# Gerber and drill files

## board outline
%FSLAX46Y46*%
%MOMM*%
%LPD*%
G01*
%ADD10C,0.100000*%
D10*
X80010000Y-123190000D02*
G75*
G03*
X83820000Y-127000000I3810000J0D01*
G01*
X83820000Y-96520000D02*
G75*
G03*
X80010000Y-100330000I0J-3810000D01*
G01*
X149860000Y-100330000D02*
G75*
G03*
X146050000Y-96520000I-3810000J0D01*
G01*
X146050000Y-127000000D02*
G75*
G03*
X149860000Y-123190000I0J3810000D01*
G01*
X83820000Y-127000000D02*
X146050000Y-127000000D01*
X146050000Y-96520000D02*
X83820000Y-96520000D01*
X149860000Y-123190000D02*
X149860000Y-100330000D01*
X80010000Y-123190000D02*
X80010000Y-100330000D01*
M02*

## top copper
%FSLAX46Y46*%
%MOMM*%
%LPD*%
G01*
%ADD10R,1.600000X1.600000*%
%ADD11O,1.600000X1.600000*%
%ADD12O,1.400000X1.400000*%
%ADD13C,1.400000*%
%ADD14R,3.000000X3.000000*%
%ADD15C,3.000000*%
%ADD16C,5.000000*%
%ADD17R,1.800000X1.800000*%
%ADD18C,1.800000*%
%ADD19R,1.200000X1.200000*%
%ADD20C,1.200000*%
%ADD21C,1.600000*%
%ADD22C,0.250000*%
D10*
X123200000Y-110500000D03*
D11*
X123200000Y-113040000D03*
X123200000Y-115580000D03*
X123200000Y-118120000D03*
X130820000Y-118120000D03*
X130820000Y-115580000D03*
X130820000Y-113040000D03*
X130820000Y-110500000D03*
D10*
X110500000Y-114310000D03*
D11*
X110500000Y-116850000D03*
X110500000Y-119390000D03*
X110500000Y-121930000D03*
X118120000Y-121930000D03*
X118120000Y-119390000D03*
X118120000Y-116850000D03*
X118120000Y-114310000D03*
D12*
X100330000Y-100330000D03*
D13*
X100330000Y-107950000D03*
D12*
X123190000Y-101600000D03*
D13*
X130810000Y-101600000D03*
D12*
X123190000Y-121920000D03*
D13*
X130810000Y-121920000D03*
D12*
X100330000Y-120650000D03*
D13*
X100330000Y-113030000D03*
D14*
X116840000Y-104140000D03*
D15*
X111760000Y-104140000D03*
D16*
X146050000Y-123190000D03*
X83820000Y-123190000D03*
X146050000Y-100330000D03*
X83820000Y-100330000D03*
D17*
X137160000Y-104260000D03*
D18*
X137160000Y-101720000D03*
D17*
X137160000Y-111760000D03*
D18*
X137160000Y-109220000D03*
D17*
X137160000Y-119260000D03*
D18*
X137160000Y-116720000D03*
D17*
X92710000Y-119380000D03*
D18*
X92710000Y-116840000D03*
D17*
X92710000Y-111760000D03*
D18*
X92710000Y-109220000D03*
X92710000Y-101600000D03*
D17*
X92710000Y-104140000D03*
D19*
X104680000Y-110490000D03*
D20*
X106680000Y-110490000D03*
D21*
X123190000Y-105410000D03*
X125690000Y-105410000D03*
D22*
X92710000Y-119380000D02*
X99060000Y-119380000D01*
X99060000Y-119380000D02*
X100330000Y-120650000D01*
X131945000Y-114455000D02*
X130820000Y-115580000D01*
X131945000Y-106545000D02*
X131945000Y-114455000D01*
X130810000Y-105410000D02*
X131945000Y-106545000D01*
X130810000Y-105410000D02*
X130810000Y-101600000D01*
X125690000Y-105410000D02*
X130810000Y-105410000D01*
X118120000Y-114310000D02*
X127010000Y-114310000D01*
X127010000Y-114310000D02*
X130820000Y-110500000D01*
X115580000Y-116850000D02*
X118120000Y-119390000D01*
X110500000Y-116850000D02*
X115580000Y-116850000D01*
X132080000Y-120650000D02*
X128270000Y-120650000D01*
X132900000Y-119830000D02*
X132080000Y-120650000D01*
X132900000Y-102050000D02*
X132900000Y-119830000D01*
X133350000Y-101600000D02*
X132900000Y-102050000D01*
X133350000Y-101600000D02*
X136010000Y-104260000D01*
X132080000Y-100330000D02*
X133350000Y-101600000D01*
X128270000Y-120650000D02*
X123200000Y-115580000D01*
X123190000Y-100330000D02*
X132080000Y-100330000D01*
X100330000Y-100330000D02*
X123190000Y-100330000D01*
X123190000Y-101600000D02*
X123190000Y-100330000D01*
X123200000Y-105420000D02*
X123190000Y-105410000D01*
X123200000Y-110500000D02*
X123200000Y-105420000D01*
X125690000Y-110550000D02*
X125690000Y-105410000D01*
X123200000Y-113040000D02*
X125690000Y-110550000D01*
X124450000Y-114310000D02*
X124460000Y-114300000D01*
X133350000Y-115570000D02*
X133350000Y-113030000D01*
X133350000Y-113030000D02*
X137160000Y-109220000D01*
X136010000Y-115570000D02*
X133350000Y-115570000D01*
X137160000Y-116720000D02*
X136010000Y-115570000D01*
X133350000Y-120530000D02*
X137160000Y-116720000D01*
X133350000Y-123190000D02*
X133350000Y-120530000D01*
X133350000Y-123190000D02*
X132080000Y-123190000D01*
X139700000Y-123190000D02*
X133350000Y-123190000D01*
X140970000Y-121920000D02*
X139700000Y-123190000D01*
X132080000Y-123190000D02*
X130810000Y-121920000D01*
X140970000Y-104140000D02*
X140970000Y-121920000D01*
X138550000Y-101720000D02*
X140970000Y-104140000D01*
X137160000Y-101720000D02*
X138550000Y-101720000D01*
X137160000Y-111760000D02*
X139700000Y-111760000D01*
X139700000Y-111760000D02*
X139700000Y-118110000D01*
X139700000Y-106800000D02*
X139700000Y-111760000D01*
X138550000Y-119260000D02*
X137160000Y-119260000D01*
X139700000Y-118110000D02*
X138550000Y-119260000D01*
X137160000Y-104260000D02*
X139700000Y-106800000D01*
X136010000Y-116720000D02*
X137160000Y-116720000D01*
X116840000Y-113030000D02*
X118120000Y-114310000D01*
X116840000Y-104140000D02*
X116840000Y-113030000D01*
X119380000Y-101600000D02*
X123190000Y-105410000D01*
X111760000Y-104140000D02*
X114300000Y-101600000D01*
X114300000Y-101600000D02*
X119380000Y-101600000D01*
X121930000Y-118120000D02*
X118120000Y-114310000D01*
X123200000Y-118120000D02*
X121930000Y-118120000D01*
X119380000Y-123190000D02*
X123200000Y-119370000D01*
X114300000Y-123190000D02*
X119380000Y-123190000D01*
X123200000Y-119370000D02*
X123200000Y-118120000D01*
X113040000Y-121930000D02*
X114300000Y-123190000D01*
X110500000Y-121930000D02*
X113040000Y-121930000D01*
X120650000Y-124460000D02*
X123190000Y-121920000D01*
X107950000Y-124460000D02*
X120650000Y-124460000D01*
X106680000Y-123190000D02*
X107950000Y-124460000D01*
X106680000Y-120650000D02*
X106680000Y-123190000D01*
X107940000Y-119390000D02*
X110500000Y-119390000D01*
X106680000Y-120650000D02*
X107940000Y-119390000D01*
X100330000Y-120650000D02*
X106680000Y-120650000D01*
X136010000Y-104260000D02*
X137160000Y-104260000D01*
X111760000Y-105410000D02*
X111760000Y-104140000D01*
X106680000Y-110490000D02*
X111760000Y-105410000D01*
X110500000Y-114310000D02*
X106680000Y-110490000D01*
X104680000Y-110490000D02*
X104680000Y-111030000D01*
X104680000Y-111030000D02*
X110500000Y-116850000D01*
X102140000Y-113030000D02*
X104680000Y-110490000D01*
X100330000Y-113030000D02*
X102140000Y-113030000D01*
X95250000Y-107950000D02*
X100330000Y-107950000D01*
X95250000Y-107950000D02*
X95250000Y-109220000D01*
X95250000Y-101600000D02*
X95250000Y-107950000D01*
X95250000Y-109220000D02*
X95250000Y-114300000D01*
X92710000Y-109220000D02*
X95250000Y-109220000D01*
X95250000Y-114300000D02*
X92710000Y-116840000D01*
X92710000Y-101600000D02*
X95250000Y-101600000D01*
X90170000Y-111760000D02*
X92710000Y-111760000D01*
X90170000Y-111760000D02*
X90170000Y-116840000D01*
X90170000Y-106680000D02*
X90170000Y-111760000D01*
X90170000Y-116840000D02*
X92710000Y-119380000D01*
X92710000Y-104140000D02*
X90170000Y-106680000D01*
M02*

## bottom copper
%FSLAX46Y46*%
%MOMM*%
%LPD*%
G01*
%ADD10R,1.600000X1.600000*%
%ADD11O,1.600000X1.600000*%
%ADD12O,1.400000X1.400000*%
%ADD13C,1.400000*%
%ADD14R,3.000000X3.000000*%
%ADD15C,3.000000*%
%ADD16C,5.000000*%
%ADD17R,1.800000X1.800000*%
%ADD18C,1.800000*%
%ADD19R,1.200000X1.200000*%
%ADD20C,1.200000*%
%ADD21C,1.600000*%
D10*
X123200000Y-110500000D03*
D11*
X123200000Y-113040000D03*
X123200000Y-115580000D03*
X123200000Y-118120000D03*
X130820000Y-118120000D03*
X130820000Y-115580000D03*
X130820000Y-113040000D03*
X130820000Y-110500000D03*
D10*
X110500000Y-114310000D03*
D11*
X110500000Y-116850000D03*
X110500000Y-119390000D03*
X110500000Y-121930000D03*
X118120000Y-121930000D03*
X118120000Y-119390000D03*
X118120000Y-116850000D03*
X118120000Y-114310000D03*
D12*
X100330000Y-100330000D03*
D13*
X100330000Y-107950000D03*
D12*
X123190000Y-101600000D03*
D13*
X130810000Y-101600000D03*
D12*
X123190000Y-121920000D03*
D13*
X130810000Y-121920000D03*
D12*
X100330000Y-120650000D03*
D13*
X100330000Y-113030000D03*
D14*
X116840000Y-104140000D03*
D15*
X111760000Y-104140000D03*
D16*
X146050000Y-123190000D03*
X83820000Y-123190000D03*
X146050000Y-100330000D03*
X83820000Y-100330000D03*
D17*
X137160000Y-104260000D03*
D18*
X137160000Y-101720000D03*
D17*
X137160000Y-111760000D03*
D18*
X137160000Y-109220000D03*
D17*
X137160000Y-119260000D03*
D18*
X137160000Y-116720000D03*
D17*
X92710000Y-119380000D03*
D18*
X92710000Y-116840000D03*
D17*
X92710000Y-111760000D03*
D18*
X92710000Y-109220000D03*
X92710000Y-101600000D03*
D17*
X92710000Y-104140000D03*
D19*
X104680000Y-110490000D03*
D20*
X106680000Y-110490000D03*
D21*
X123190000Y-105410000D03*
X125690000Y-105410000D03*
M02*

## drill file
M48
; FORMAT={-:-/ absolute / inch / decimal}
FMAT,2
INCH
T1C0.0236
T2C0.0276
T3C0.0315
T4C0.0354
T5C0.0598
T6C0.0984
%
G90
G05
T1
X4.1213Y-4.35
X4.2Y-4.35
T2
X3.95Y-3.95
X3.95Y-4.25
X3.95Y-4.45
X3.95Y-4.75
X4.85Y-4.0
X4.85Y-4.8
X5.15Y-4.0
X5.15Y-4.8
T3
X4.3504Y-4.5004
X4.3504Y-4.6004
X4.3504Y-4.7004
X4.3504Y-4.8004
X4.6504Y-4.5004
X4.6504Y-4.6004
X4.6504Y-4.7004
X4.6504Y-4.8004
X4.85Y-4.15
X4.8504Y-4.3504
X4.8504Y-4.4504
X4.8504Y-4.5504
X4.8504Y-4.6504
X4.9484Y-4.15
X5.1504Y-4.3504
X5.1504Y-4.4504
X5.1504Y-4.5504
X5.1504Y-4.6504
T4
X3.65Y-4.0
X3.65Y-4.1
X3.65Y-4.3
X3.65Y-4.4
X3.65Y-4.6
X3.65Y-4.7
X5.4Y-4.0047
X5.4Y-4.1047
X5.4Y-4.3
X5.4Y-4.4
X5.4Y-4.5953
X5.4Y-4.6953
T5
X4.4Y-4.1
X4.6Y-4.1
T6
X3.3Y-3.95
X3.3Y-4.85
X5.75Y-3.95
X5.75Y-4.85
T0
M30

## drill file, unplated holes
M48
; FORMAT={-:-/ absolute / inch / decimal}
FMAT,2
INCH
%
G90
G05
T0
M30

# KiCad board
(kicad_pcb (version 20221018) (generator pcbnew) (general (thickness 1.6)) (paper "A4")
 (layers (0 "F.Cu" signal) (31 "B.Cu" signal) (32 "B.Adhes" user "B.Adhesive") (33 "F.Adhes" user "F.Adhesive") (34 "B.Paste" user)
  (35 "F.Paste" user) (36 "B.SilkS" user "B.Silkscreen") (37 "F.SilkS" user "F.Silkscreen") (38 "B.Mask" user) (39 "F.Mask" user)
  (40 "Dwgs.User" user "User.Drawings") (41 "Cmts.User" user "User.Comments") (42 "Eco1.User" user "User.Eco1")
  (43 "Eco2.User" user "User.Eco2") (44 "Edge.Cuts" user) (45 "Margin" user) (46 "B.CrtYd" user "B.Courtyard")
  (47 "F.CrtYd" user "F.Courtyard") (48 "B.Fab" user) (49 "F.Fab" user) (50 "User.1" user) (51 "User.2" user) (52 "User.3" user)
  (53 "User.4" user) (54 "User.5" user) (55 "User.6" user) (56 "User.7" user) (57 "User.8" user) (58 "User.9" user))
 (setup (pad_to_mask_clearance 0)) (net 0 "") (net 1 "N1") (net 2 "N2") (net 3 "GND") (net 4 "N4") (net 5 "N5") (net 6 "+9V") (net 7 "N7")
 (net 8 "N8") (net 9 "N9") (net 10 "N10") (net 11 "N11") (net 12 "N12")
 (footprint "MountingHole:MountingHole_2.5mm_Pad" (layer "F.Cu") (at 83.82 100.33)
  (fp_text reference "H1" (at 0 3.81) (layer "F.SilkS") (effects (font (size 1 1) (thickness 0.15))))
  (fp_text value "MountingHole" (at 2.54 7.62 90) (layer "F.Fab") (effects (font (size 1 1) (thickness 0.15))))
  (pad "1" thru_hole circle (at 0 0) (size 5 5) (drill 2.5) (layers "*.Cu" "*.Mask")))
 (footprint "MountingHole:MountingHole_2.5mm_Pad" (layer "F.Cu") (at 146.05 123.19)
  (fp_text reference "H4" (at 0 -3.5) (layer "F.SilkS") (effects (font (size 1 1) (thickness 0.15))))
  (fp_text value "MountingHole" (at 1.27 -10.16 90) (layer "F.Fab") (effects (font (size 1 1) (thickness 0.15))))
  (pad "1" thru_hole circle (at 0 0) (size 5 5) (drill 2.5) (layers "*.Cu" "*.Mask")))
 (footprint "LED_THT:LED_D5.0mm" (layer "F.Cu") (at 137.16 104.26 90)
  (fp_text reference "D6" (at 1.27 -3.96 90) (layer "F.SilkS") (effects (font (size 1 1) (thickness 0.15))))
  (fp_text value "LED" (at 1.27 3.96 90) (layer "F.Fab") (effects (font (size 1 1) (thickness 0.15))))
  (pad "1" thru_hole rect (at 0 0 90) (size 1.8 1.8) (drill 0.9) (layers "*.Cu" "*.Mask") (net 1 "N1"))
  (pad "2" thru_hole circle (at 2.54 0 90) (size 1.8 1.8) (drill 0.9) (layers "*.Cu" "*.Mask") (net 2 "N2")))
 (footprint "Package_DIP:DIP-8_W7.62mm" (layer "F.Cu") (at 110.5 114.31)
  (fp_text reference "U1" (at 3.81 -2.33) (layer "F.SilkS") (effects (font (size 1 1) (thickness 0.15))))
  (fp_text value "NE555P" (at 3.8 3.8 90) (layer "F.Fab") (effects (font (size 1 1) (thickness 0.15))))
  (pad "1" thru_hole rect (at 0 0) (size 1.6 1.6) (drill 0.8) (layers "*.Cu" "*.Mask") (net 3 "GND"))
  (pad "2" thru_hole oval (at 0 2.54) (size 1.6 1.6) (drill 0.8) (layers "*.Cu" "*.Mask") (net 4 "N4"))
  (pad "3" thru_hole oval (at 0 5.08) (size 1.6 1.6) (drill 0.8) (layers "*.Cu" "*.Mask") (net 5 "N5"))
  (pad "4" thru_hole oval (at 0 7.62) (size 1.6 1.6) (drill 0.8) (layers "*.Cu" "*.Mask") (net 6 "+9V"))
  (pad "5" thru_hole oval (at 7.62 7.62) (size 1.6 1.6) (drill 0.8) (layers "*.Cu" "*.Mask") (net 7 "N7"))
  (pad "6" thru_hole oval (at 7.62 5.08) (size 1.6 1.6) (drill 0.8) (layers "*.Cu" "*.Mask") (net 4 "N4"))
  (pad "7" thru_hole oval (at 7.62 2.54) (size 1.6 1.6) (drill 0.8) (layers "*.Cu" "*.Mask") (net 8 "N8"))
  (pad "8" thru_hole oval (at 7.62 0) (size 1.6 1.6) (drill 0.8) (layers "*.Cu" "*.Mask") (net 6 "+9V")))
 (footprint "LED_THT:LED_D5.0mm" (layer "F.Cu") (at 92.71 104.14 90)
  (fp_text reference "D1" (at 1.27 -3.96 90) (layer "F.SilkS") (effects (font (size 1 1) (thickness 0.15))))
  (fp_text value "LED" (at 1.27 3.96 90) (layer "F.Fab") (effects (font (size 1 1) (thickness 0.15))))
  (pad "1" thru_hole rect (at 0 0 90) (size 1.8 1.8) (drill 0.9) (layers "*.Cu" "*.Mask") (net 5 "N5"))
  (pad "2" thru_hole circle (at 2.54 0 90) (size 1.8 1.8) (drill 0.9) (layers "*.Cu" "*.Mask") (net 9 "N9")))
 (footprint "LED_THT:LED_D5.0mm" (layer "F.Cu") (at 92.71 119.38 90)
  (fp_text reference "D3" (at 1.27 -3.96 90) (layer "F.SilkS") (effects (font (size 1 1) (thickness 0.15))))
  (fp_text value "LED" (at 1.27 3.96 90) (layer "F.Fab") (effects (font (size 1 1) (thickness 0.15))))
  (pad "1" thru_hole rect (at 0 0 90) (size 1.8 1.8) (drill 0.9) (layers "*.Cu" "*.Mask") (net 5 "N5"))
  (pad "2" thru_hole circle (at 2.54 0 90) (size 1.8 1.8) (drill 0.9) (layers "*.Cu" "*.Mask") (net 9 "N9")))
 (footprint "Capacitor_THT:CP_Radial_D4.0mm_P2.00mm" (layer "F.Cu") (at 104.68 110.49)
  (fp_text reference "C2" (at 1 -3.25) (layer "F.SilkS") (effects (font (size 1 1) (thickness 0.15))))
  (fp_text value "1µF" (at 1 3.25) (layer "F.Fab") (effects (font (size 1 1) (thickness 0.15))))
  (pad "1" thru_hole rect (at 0 0) (size 1.2 1.2) (drill 0.6) (layers "*.Cu" "*.Mask") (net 4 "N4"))
  (pad "2" thru_hole circle (at 2 0) (size 1.2 1.2) (drill 0.6) (layers "*.Cu" "*.Mask") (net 3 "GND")))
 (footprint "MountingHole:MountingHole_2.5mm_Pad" (layer "F.Cu") (at 83.82 123.19)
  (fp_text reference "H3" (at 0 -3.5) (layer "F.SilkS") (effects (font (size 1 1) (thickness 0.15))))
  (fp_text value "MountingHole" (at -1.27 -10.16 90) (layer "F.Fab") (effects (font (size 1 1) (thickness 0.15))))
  (pad "1" thru_hole circle (at 0 0) (size 5 5) (drill 2.5) (layers "*.Cu" "*.Mask")))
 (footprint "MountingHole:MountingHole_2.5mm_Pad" (layer "F.Cu") (at 146.05 100.33)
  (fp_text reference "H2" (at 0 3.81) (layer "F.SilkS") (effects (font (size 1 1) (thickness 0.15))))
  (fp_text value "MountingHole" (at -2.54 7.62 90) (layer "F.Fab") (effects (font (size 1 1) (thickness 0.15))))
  (pad "1" thru_hole circle (at 0 0) (size 5 5) (drill 2.5) (layers "*.Cu" "*.Mask")))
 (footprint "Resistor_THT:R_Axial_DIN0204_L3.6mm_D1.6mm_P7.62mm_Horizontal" (layer "F.Cu") (at 100.33 113.03 -90)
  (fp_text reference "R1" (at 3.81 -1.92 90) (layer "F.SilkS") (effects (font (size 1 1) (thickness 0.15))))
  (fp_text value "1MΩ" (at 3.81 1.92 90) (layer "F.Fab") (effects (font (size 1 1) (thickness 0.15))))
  (pad "1" thru_hole circle (at 0 0 270) (size 1.4 1.4) (drill 0.7) (layers "*.Cu" "*.Mask") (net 4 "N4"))
  (pad "2" thru_hole oval (at 7.62 0 270) (size 1.4 1.4) (drill 0.7) (layers "*.Cu" "*.Mask") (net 5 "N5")))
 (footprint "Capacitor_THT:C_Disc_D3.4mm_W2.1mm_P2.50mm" (layer "F.Cu") (at 125.69 105.41 180)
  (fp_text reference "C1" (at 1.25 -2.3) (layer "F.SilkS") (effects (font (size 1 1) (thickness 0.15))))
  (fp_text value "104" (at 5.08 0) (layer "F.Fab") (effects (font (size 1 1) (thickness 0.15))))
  (pad "1" thru_hole circle (at 0 0 180) (size 1.6 1.6) (drill 0.8) (layers "*.Cu" "*.Mask") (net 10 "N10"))
  (pad "2" thru_hole circle (at 2.5 0 180) (size 1.6 1.6) (drill 0.8) (layers "*.Cu" "*.Mask") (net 3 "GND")))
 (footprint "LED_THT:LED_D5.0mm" (layer "F.Cu") (at 92.71 111.76 90)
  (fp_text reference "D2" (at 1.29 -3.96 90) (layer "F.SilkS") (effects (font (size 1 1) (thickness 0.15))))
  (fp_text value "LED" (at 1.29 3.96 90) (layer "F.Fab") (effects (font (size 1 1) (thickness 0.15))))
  (pad "1" thru_hole rect (at 0 0 90) (size 1.8 1.8) (drill 0.9) (layers "*.Cu" "*.Mask") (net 5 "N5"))
  (pad "2" thru_hole circle (at 2.54 0 90) (size 1.8 1.8) (drill 0.9) (layers "*.Cu" "*.Mask") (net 9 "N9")))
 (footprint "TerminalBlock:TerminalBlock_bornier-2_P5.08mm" (layer "F.Cu") (at 116.84 104.14 180)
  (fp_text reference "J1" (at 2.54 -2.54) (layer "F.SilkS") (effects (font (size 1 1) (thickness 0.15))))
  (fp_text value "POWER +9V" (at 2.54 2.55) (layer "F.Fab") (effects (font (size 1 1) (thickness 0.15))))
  (pad "1" thru_hole rect (at 0 0 180) (size 3 3) (drill 1.52) (layers "*.Cu" "*.Mask") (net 6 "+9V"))
  (pad "2" thru_hole circle (at 5.08 0 180) (size 3 3) (drill 1.52) (layers "*.Cu" "*.Mask") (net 3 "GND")))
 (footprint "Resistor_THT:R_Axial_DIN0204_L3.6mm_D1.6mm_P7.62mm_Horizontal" (layer "F.Cu") (at 100.33 107.95 90)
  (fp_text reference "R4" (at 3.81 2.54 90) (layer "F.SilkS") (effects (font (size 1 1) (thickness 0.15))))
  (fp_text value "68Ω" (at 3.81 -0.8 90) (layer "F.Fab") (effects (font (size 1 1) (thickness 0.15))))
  (pad "1" thru_hole circle (at 0 0 90) (size 1.4 1.4) (drill 0.7) (layers "*.Cu" "*.Mask") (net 9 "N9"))
  (pad "2" thru_hole oval (at 7.62 0 90) (size 1.4 1.4) (drill 0.7) (layers "*.Cu" "*.Mask") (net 1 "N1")))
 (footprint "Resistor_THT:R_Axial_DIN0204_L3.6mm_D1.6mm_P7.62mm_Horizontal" (layer "F.Cu") (at 130.81 101.6 180)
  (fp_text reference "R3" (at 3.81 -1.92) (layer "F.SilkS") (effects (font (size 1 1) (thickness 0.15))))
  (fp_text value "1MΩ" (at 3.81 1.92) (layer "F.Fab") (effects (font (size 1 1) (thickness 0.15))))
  (pad "1" thru_hole circle (at 0 0 180) (size 1.4 1.4) (drill 0.7) (layers "*.Cu" "*.Mask") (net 10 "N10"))
  (pad "2" thru_hole oval (at 7.62 0 180) (size 1.4 1.4) (drill 0.7) (layers "*.Cu" "*.Mask") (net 1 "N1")))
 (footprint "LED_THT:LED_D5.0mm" (layer "F.Cu") (at 137.16 119.26 90)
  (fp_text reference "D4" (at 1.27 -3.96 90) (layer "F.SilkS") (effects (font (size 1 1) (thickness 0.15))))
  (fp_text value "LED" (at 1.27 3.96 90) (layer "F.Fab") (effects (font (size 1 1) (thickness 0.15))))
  (pad "1" thru_hole rect (at 0 0 90) (size 1.8 1.8) (drill 0.9) (layers "*.Cu" "*.Mask") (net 1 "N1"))
  (pad "2" thru_hole circle (at 2.54 0 90) (size 1.8 1.8) (drill 0.9) (layers "*.Cu" "*.Mask") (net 2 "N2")))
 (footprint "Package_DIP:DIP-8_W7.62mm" (layer "F.Cu") (at 123.2 110.5)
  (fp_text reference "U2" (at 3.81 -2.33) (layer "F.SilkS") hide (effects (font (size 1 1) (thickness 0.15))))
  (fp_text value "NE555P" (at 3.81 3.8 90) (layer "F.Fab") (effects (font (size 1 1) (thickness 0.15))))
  (pad "1" thru_hole rect (at 0 0) (size 1.6 1.6) (drill 0.8) (layers "*.Cu" "*.Mask") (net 3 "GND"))
  (pad "2" thru_hole oval (at 0 2.54) (size 1.6 1.6) (drill 0.8) (layers "*.Cu" "*.Mask") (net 10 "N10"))
  (pad "3" thru_hole oval (at 0 5.08) (size 1.6 1.6) (drill 0.8) (layers "*.Cu" "*.Mask") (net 1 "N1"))
  (pad "4" thru_hole oval (at 0 7.62) (size 1.6 1.6) (drill 0.8) (layers "*.Cu" "*.Mask") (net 6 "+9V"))
  (pad "5" thru_hole oval (at 7.62 7.62) (size 1.6 1.6) (drill 0.8) (layers "*.Cu" "*.Mask") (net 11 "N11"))
  (pad "6" thru_hole oval (at 7.62 5.08) (size 1.6 1.6) (drill 0.8) (layers "*.Cu" "*.Mask") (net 10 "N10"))
  (pad "7" thru_hole oval (at 7.62 2.54) (size 1.6 1.6) (drill 0.8) (layers "*.Cu" "*.Mask") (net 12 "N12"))
  (pad "8" thru_hole oval (at 7.62 0) (size 1.6 1.6) (drill 0.8) (layers "*.Cu" "*.Mask") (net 6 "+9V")))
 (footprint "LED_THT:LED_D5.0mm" (layer "F.Cu") (at 137.16 111.76 90)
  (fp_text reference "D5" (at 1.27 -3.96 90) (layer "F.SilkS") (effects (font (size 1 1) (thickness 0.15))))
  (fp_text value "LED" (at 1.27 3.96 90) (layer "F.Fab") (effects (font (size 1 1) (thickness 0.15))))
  (pad "1" thru_hole rect (at 0 0 90) (size 1.8 1.8) (drill 0.9) (layers "*.Cu" "*.Mask") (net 1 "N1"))
  (pad "2" thru_hole circle (at 2.54 0 90) (size 1.8 1.8) (drill 0.9) (layers "*.Cu" "*.Mask") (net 2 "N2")))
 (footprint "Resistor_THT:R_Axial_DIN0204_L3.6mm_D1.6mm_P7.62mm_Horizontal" (layer "F.Cu") (at 130.81 121.92 180)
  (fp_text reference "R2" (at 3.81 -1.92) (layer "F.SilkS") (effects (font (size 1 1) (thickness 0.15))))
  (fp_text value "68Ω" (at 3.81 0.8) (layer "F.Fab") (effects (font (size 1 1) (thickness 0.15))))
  (pad "1" thru_hole circle (at 0 0 180) (size 1.4 1.4) (drill 0.7) (layers "*.Cu" "*.Mask") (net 2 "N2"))
  (pad "2" thru_hole oval (at 7.62 0 180) (size 1.4 1.4) (drill 0.7) (layers "*.Cu" "*.Mask") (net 5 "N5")))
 (gr_line (start 149.86 123.19) (end 149.86 100.33) (stroke (width 0.1) (type default)) (layer "Edge.Cuts"))
 (gr_arc (start 80.01 100.33) (mid 81.125923 97.635923) (end 83.82 96.52) (stroke (width 0.1) (type default)) (layer "Edge.Cuts"))
 (gr_arc (start 146.05 96.52) (mid 148.744077 97.635923) (end 149.86 100.33) (stroke (width 0.1) (type default)) (layer "Edge.Cuts"))
 (gr_line (start 146.05 96.52) (end 83.82 96.52) (stroke (width 0.1) (type default)) (layer "Edge.Cuts"))
 (gr_arc (start 149.86 123.19) (mid 148.744077 125.884077) (end 146.05 127) (stroke (width 0.1) (type default)) (layer "Edge.Cuts"))
 (gr_arc (start 83.82 127) (mid 81.125923 125.884077) (end 80.01 123.19) (stroke (width 0.1) (type default)) (layer "Edge.Cuts"))
 (gr_line (start 80.01 123.19) (end 80.01 100.33) (stroke (width 0.1) (type default)) (layer "Edge.Cuts"))
 (gr_line (start 83.82 127) (end 146.05 127) (stroke (width 0.1) (type default)) (layer "Edge.Cuts"))
 (segment (start 123.2 113.04) (end 125.69 110.55) (width 0.25) (layer "F.Cu") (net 10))
 (segment (start 130.81 105.41) (end 130.81 101.6) (width 0.25) (layer "F.Cu") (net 10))
 (segment (start 125.69 110.55) (end 125.69 105.41) (width 0.25) (layer "F.Cu") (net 10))
 (segment (start 125.69 105.41) (end 130.81 105.41) (width 0.25) (layer "F.Cu") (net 10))
 (segment (start 131.945 106.545) (end 131.945 114.455) (width 0.25) (layer "F.Cu") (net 10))
 (segment (start 130.81 105.41) (end 131.945 106.545) (width 0.25) (layer "F.Cu") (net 10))
 (segment (start 131.945 114.455) (end 130.82 115.58) (width 0.25) (layer "F.Cu") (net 10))
 (segment (start 111.76 105.41) (end 111.76 104.14) (width 0.25) (layer "F.Cu") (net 3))
 (segment (start 110.5 114.31) (end 106.68 110.49) (width 0.25) (layer "F.Cu") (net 3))
 (segment (start 123.2 105.42) (end 123.19 105.41) (width 0.25) (layer "F.Cu") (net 3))
 (segment (start 123.2 110.5) (end 123.2 105.42) (width 0.25) (layer "F.Cu") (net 3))
 (segment (start 114.3 101.6) (end 119.38 101.6) (width 0.25) (layer "F.Cu") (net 3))
 (segment (start 111.76 104.14) (end 114.3 101.6) (width 0.25) (layer "F.Cu") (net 3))
 (segment (start 119.38 101.6) (end 123.19 105.41) (width 0.25) (layer "F.Cu") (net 3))
 (segment (start 106.68 110.49) (end 111.76 105.41) (width 0.25) (layer "F.Cu") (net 3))
 (segment (start 115.58 116.85) (end 118.12 119.39) (width 0.25) (layer "F.Cu") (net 4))
 (segment (start 102.14 113.03) (end 104.68 110.49) (width 0.25) (layer "F.Cu") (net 4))
 (segment (start 100.33 113.03) (end 102.14 113.03) (width 0.25) (layer "F.Cu") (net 4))
 (segment (start 104.68 111.03) (end 110.5 116.85) (width 0.25) (layer "F.Cu") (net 4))
 (segment (start 104.68 110.49) (end 104.68 111.03) (width 0.25) (layer "F.Cu") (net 4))
 (segment (start 110.5 116.85) (end 115.58 116.85) (width 0.25) (layer "F.Cu") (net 4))
 (segment (start 90.17 106.68) (end 90.17 111.76) (width 0.25) (layer "F.Cu") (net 5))
 (segment (start 90.17 116.84) (end 92.71 119.38) (width 0.25) (layer "F.Cu") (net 5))
 (segment (start 90.17 111.76) (end 90.17 116.84) (width 0.25) (layer "F.Cu") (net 5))
 (segment (start 107.94 119.39) (end 110.5 119.39) (width 0.25) (layer "F.Cu") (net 5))
 (segment (start 120.65 124.46) (end 123.19 121.92) (width 0.25) (layer "F.Cu") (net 5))
 (segment (start 106.68 120.65) (end 106.68 123.19) (width 0.25) (layer "F.Cu") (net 5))
 (segment (start 92.71 119.38) (end 99.06 119.38) (width 0.25) (layer "F.Cu") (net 5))
 (segment (start 106.68 123.19) (end 107.95 124.46) (width 0.25) (layer "F.Cu") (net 5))
 (segment (start 107.95 124.46) (end 120.65 124.46) (width 0.25) (layer "F.Cu") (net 5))
 (segment (start 99.06 119.38) (end 100.33 120.65) (width 0.25) (layer "F.Cu") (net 5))
 (segment (start 92.71 104.14) (end 90.17 106.68) (width 0.25) (layer "F.Cu") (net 5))
 (segment (start 106.68 120.65) (end 107.94 119.39) (width 0.25) (layer "F.Cu") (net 5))
 (segment (start 100.33 120.65) (end 106.68 120.65) (width 0.25) (layer "F.Cu") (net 5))
 (segment (start 90.17 111.76) (end 92.71 111.76) (width 0.25) (layer "F.Cu") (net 5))
 (segment (start 95.25 109.22) (end 95.25 114.3) (width 0.25) (layer "F.Cu") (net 9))
 (segment (start 95.25 107.95) (end 95.25 109.22) (width 0.25) (layer "F.Cu") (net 9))
 (segment (start 95.25 114.3) (end 92.71 116.84) (width 0.25) (layer "F.Cu") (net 9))
 (segment (start 92.71 109.22) (end 95.25 109.22) (width 0.25) (layer "F.Cu") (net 9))
 (segment (start 92.71 101.6) (end 95.25 101.6) (width 0.25) (layer "F.Cu") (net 9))
 (segment (start 95.25 107.95) (end 100.33 107.95) (width 0.25) (layer "F.Cu") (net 9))
 (segment (start 95.25 101.6) (end 95.25 107.95) (width 0.25) (layer "F.Cu") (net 9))
 (segment (start 133.35 101.6) (end 132.9 102.05) (width 0.25) (layer "F.Cu") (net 1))
 (segment (start 123.19 100.33) (end 132.08 100.33) (width 0.25) (layer "F.Cu") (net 1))
 (segment (start 137.16 111.76) (end 139.7 111.76) (width 0.25) (layer "F.Cu") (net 1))
 (segment (start 132.08 100.33) (end 133.35 101.6) (width 0.25) (layer "F.Cu") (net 1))
 (segment (start 139.7 106.8) (end 139.7 111.76) (width 0.25) (layer "F.Cu") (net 1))
 (segment (start 139.7 111.76) (end 139.7 118.11) (width 0.25) (layer "F.Cu") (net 1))
 (segment (start 132.08 120.65) (end 128.27 120.65) (width 0.25) (layer "F.Cu") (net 1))
 (segment (start 138.55 119.26) (end 137.16 119.26) (width 0.25) (layer "F.Cu") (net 1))
 (segment (start 132.9 119.83) (end 132.08 120.65) (width 0.25) (layer "F.Cu") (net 1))
 (segment (start 128.27 120.65) (end 123.2 115.58) (width 0.25) (layer "F.Cu") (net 1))
 (segment (start 137.16 104.26) (end 139.7 106.8) (width 0.25) (layer "F.Cu") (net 1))
 (segment (start 132.9 102.05) (end 132.9 119.83) (width 0.25) (layer "F.Cu") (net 1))
 (segment (start 100.33 100.33) (end 123.19 100.33) (width 0.25) (layer "F.Cu") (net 1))
 (segment (start 136.01 104.26) (end 137.16 104.26) (width 0.25) (layer "F.Cu") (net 1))
 (segment (start 133.35 101.6) (end 136.01 104.26) (width 0.25) (layer "F.Cu") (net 1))
 (segment (start 123.19 101.6) (end 123.19 100.33) (width 0.25) (layer "F.Cu") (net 1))
 (segment (start 139.7 118.11) (end 138.55 119.26) (width 0.25) (layer "F.Cu") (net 1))
 (segment (start 133.35 113.03) (end 137.16 109.22) (width 0.25) (layer "F.Cu") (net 2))
 (segment (start 136.01 115.57) (end 133.35 115.57) (width 0.25) (layer "F.Cu") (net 2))
 (segment (start 132.08 123.19) (end 130.81 121.92) (width 0.25) (layer "F.Cu") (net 2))
 (segment (start 138.55 101.72) (end 140.97 104.14) (width 0.25) (layer "F.Cu") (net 2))
 (segment (start 137.16 116.72) (end 136.01 115.57) (width 0.25) (layer "F.Cu") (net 2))
 (segment (start 133.35 115.57) (end 133.35 113.03) (width 0.25) (layer "F.Cu") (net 2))
 (segment (start 133.35 120.53) (end 137.16 116.72) (width 0.25) (layer "F.Cu") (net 2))
 (segment (start 140.97 104.14) (end 140.97 121.92) (width 0.25) (layer "F.Cu") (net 2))
 (segment (start 136.01 116.72) (end 137.16 116.72) (width 0.25) (layer "F.Cu") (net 2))
 (segment (start 137.16 101.72) (end 138.55 101.72) (width 0.25) (layer "F.Cu") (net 2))
 (segment (start 139.7 123.19) (end 133.35 123.19) (width 0.25) (layer "F.Cu") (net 2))
 (segment (start 133.35 123.19) (end 132.08 123.19) (width 0.25) (layer "F.Cu") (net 2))
 (segment (start 140.97 121.92) (end 139.7 123.19) (width 0.25) (layer "F.Cu") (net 2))
 (segment (start 133.35 123.19) (end 133.35 120.53) (width 0.25) (layer "F.Cu") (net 2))
 (segment (start 116.84 113.03) (end 118.12 114.31) (width 0.25) (layer "F.Cu") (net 6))
 (segment (start 114.3 123.19) (end 119.38 123.19) (width 0.25) (layer "F.Cu") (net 6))
 (segment (start 110.5 121.93) (end 113.04 121.93) (width 0.25) (layer "F.Cu") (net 6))
 (segment (start 116.84 104.14) (end 116.84 113.03) (width 0.25) (layer "F.Cu") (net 6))
 (segment (start 124.45 114.31) (end 124.46 114.3) (width 0.25) (layer "F.Cu") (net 6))
 (segment (start 127.01 114.31) (end 130.82 110.5) (width 0.25) (layer "F.Cu") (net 6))
 (segment (start 123.2 119.37) (end 123.2 118.12) (width 0.25) (layer "F.Cu") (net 6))
 (segment (start 121.93 118.12) (end 118.12 114.31) (width 0.25) (layer "F.Cu") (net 6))
 (segment (start 113.04 121.93) (end 114.3 123.19) (width 0.25) (layer "F.Cu") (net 6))
 (segment (start 118.12 114.31) (end 127.01 114.31) (width 0.25) (layer "F.Cu") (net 6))
 (segment (start 119.38 123.19) (end 123.2 119.37) (width 0.25) (layer "F.Cu") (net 6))
 (segment (start 123.2 118.12) (end 121.93 118.12) (width 0.25) (layer "F.Cu") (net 6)))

